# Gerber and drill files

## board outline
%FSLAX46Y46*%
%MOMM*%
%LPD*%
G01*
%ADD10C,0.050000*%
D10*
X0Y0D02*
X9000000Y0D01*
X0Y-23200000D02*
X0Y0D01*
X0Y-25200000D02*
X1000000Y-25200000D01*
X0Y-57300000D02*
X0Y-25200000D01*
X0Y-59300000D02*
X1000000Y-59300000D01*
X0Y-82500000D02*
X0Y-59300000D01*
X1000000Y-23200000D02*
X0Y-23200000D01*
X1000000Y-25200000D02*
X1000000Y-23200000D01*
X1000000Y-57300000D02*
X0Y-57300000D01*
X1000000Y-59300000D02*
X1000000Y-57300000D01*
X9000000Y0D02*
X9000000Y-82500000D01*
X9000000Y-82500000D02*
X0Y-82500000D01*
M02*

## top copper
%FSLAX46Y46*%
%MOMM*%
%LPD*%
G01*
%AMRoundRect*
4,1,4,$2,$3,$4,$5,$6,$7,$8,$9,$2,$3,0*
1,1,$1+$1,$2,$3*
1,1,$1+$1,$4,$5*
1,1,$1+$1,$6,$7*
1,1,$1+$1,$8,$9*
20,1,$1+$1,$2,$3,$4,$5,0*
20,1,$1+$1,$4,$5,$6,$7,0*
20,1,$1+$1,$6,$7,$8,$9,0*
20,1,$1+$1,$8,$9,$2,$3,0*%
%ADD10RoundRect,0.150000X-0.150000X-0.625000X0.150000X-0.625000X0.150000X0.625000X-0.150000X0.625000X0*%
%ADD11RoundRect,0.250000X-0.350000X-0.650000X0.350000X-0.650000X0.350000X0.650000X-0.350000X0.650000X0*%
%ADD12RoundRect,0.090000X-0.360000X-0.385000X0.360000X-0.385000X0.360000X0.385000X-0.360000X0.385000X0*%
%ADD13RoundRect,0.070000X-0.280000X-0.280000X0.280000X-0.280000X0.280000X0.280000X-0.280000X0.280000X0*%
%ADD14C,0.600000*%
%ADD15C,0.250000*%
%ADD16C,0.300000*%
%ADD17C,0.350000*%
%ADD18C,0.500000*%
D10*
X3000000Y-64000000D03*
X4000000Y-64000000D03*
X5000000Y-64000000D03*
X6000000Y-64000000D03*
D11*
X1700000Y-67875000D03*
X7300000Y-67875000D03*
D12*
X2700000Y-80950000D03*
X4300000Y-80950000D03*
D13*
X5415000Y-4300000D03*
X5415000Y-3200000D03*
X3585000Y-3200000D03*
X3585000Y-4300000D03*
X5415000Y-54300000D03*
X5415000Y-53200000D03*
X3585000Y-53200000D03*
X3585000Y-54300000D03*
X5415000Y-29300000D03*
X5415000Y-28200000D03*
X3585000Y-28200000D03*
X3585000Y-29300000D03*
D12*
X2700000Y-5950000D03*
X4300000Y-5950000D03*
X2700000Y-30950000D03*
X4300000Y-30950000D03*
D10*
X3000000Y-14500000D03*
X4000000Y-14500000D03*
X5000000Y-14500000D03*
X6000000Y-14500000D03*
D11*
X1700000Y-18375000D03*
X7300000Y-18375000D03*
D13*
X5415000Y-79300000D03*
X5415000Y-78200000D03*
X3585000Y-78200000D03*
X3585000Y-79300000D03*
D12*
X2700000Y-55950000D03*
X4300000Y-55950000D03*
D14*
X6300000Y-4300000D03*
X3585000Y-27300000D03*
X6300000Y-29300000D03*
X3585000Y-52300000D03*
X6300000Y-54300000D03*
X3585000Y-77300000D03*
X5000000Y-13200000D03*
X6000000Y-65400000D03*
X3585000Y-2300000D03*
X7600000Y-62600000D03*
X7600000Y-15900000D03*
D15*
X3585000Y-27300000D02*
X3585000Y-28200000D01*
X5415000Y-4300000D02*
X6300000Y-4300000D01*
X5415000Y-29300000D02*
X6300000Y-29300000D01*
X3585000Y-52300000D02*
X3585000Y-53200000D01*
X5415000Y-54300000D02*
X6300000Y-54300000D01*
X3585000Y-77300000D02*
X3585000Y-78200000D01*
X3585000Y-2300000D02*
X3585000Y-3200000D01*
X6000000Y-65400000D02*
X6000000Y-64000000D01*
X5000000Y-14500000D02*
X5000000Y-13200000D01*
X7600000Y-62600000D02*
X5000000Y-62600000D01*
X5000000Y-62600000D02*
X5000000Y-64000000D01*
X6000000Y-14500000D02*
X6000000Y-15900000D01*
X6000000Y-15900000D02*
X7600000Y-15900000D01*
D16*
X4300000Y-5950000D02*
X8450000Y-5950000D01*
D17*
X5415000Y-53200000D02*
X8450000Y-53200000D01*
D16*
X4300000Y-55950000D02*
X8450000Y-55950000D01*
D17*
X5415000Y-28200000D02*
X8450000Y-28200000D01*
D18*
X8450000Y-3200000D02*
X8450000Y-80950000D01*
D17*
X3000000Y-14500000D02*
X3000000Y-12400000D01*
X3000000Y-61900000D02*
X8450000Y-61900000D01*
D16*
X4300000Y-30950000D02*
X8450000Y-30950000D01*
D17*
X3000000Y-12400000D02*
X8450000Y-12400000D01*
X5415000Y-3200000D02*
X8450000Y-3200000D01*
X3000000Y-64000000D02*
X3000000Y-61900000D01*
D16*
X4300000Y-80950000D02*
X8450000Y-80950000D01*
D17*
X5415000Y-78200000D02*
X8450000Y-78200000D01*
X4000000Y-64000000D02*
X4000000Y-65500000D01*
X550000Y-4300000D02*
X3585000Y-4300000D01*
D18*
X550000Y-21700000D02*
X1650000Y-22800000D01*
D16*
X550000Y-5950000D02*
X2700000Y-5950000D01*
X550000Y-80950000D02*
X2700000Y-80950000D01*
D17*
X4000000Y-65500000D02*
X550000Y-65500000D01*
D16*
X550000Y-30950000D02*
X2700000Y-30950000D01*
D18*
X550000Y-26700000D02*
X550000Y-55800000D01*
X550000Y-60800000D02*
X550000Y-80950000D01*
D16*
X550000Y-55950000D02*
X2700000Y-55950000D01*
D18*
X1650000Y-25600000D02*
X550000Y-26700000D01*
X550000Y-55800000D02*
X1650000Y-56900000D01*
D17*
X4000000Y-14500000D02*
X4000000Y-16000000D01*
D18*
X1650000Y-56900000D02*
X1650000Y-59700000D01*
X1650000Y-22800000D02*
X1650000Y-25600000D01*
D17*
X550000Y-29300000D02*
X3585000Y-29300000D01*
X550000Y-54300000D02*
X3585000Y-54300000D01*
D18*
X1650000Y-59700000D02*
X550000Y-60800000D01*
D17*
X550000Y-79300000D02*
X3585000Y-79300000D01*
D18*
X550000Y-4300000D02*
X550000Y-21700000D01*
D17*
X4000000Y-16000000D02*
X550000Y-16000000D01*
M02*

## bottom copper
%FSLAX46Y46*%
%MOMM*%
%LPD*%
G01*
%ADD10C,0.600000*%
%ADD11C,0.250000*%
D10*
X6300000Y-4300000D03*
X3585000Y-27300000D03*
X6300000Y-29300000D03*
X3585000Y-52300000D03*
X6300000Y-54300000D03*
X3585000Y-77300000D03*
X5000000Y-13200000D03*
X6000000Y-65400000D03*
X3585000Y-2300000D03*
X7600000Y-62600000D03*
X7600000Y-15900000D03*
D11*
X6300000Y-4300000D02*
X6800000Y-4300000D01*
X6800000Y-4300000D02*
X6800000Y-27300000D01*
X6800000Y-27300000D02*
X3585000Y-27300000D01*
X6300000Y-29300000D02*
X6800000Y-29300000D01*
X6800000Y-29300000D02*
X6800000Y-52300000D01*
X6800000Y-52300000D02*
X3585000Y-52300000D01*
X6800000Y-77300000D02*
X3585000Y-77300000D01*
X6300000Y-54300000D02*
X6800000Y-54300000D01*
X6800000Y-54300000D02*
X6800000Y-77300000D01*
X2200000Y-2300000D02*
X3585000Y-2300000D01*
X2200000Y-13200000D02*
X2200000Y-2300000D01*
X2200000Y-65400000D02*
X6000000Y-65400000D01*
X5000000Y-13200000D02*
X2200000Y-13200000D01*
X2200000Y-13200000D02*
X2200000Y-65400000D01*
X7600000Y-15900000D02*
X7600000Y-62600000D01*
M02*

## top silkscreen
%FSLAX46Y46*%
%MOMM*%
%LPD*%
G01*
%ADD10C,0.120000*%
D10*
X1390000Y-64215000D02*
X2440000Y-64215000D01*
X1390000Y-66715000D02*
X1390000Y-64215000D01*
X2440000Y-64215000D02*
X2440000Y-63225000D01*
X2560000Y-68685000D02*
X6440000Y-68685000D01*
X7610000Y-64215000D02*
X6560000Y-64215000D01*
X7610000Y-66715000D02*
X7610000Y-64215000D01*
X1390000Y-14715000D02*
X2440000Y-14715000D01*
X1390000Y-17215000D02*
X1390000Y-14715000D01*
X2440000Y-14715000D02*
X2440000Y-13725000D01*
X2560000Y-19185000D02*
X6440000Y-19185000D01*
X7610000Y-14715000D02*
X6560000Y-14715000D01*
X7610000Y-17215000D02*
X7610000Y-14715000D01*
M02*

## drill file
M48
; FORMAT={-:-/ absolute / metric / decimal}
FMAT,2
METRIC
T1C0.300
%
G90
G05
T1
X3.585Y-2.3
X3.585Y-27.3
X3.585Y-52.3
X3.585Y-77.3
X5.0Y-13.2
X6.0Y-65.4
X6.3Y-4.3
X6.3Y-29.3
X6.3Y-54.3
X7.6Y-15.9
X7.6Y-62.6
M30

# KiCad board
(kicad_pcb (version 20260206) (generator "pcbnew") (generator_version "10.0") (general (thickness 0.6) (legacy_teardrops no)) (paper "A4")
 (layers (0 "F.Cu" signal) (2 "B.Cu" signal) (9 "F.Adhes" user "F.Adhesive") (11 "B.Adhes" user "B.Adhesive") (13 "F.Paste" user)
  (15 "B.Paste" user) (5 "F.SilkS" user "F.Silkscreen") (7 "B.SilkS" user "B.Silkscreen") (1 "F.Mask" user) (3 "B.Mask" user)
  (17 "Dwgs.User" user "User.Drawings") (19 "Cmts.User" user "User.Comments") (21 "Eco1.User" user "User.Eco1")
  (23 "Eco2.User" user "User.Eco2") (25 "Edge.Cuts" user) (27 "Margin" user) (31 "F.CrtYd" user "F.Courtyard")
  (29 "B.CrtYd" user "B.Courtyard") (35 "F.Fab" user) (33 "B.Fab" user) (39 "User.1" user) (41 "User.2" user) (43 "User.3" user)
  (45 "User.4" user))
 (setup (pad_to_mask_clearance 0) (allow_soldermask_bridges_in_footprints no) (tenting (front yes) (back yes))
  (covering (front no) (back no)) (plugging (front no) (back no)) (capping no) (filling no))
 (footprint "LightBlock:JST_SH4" (layer "F.Cu") (at 4.5 66)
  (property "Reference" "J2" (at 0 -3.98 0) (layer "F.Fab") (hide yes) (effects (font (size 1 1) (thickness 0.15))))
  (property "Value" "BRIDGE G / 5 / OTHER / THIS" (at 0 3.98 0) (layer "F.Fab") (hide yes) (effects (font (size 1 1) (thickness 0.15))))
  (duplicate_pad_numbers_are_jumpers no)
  (fp_line (start -3.11 -1.785) (end -2.06 -1.785) (stroke (width 0.12) (type solid)) (layer "F.SilkS"))
  (fp_line (start -3.11 0.715) (end -3.11 -1.785) (stroke (width 0.12) (type solid)) (layer "F.SilkS"))
  (fp_line (start -2.06 -1.785) (end -2.06 -2.775) (stroke (width 0.12) (type solid)) (layer "F.SilkS"))
  (fp_line (start -1.94 2.685) (end 1.94 2.685) (stroke (width 0.12) (type solid)) (layer "F.SilkS"))
  (fp_line (start 3.11 -1.785) (end 2.06 -1.785) (stroke (width 0.12) (type solid)) (layer "F.SilkS"))
  (fp_line (start 3.11 0.715) (end 3.11 -1.785) (stroke (width 0.12) (type solid)) (layer "F.SilkS"))
  (pad "1" smd roundrect (at -1.5 -2) (size 0.6 1.55) (layers "F.Cu" "F.Mask" "F.Paste") (roundrect_rratio 0.25) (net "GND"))
  (pad "2" smd roundrect (at -0.5 -2) (size 0.6 1.55) (layers "F.Cu" "F.Mask" "F.Paste") (roundrect_rratio 0.25) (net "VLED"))
  (pad "3" smd roundrect (at 0.5 -2) (size 0.6 1.55) (layers "F.Cu" "F.Mask" "F.Paste") (roundrect_rratio 0.25) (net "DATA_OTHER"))
  (pad "4" smd roundrect (at 1.5 -2) (size 0.6 1.55) (layers "F.Cu" "F.Mask" "F.Paste") (roundrect_rratio 0.25) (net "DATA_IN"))
  (pad "MP" smd roundrect (at -2.8 1.875) (size 1.2 1.8) (layers "F.Cu" "F.Mask" "F.Paste") (roundrect_rratio 0.208333))
  (pad "MP" smd roundrect (at 2.8 1.875) (size 1.2 1.8) (layers "F.Cu" "F.Mask" "F.Paste") (roundrect_rratio 0.208333)))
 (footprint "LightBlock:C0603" (layer "F.Cu") (at 3.5 80.95)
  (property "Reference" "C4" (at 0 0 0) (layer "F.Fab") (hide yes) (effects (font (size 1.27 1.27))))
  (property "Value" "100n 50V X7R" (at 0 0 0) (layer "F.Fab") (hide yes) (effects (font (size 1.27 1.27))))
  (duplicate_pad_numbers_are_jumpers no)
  (pad "1" smd roundrect (at -0.8 0) (size 0.9 0.95) (layers "F.Cu" "F.Mask" "F.Paste") (roundrect_rratio 0.1) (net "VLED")
   (thermal_bridge_angle 45))
  (pad "2" smd roundrect (at 0.8 0) (size 0.9 0.95) (layers "F.Cu" "F.Mask" "F.Paste") (roundrect_rratio 0.1) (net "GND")
   (thermal_bridge_angle 45)))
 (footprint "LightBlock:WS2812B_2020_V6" (layer "F.Cu") (at 4.5 3.75)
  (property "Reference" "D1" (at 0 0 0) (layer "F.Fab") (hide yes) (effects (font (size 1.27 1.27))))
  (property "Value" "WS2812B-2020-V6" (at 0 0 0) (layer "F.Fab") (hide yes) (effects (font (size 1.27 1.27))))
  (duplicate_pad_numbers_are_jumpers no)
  (pad "1" smd roundrect (at 0.915 0.55) (size 0.7 0.7) (layers "F.Cu" "F.Mask" "F.Paste") (roundrect_rratio 0.1) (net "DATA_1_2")
   (thermal_bridge_angle 45))
  (pad "2" smd roundrect (at 0.915 -0.55) (size 0.7 0.7) (layers "F.Cu" "F.Mask" "F.Paste") (roundrect_rratio 0.1) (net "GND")
   (thermal_bridge_angle 45))
  (pad "3" smd roundrect (at -0.915 -0.55) (size 0.7 0.7) (layers "F.Cu" "F.Mask" "F.Paste") (roundrect_rratio 0.1) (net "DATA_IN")
   (thermal_bridge_angle 45))
  (pad "4" smd roundrect (at -0.915 0.55) (size 0.7 0.7) (layers "F.Cu" "F.Mask" "F.Paste") (roundrect_rratio 0.1) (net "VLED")
   (thermal_bridge_angle 45)))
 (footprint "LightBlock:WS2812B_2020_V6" (layer "F.Cu") (at 4.5 53.75)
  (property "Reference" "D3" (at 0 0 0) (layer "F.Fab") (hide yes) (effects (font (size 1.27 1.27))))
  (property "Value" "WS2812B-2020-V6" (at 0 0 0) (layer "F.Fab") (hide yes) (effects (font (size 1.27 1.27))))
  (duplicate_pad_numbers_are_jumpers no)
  (pad "1" smd roundrect (at 0.915 0.55) (size 0.7 0.7) (layers "F.Cu" "F.Mask" "F.Paste") (roundrect_rratio 0.1) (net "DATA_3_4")
   (thermal_bridge_angle 45))
  (pad "2" smd roundrect (at 0.915 -0.55) (size 0.7 0.7) (layers "F.Cu" "F.Mask" "F.Paste") (roundrect_rratio 0.1) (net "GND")
   (thermal_bridge_angle 45))
  (pad "3" smd roundrect (at -0.915 -0.55) (size 0.7 0.7) (layers "F.Cu" "F.Mask" "F.Paste") (roundrect_rratio 0.1) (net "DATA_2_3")
   (thermal_bridge_angle 45))
  (pad "4" smd roundrect (at -0.915 0.55) (size 0.7 0.7) (layers "F.Cu" "F.Mask" "F.Paste") (roundrect_rratio 0.1) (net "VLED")
   (thermal_bridge_angle 45)))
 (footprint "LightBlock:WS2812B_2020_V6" (layer "F.Cu") (at 4.5 28.75)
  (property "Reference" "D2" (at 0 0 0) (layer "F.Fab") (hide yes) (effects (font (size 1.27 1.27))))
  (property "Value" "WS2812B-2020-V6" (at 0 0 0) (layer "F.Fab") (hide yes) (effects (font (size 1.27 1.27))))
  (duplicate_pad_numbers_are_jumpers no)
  (pad "1" smd roundrect (at 0.915 0.55) (size 0.7 0.7) (layers "F.Cu" "F.Mask" "F.Paste") (roundrect_rratio 0.1) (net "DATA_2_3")
   (thermal_bridge_angle 45))
  (pad "2" smd roundrect (at 0.915 -0.55) (size 0.7 0.7) (layers "F.Cu" "F.Mask" "F.Paste") (roundrect_rratio 0.1) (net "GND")
   (thermal_bridge_angle 45))
  (pad "3" smd roundrect (at -0.915 -0.55) (size 0.7 0.7) (layers "F.Cu" "F.Mask" "F.Paste") (roundrect_rratio 0.1) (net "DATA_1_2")
   (thermal_bridge_angle 45))
  (pad "4" smd roundrect (at -0.915 0.55) (size 0.7 0.7) (layers "F.Cu" "F.Mask" "F.Paste") (roundrect_rratio 0.1) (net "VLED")
   (thermal_bridge_angle 45)))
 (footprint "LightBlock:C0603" (layer "F.Cu") (at 3.5 5.95)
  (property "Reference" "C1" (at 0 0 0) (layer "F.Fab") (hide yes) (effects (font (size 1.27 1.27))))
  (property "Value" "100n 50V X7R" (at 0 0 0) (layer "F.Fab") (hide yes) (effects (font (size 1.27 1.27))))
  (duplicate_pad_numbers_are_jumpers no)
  (pad "1" smd roundrect (at -0.8 0) (size 0.9 0.95) (layers "F.Cu" "F.Mask" "F.Paste") (roundrect_rratio 0.1) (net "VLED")
   (thermal_bridge_angle 45))
  (pad "2" smd roundrect (at 0.8 0) (size 0.9 0.95) (layers "F.Cu" "F.Mask" "F.Paste") (roundrect_rratio 0.1) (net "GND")
   (thermal_bridge_angle 45)))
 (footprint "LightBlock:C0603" (layer "F.Cu") (at 3.5 30.95)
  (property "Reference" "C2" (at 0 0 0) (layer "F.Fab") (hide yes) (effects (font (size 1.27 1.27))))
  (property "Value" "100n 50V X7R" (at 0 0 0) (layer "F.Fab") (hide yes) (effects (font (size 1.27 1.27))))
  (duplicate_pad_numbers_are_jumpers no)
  (pad "1" smd roundrect (at -0.8 0) (size 0.9 0.95) (layers "F.Cu" "F.Mask" "F.Paste") (roundrect_rratio 0.1) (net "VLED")
   (thermal_bridge_angle 45))
  (pad "2" smd roundrect (at 0.8 0) (size 0.9 0.95) (layers "F.Cu" "F.Mask" "F.Paste") (roundrect_rratio 0.1) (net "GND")
   (thermal_bridge_angle 45)))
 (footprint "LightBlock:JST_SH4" (layer "F.Cu") (at 4.5 16.5)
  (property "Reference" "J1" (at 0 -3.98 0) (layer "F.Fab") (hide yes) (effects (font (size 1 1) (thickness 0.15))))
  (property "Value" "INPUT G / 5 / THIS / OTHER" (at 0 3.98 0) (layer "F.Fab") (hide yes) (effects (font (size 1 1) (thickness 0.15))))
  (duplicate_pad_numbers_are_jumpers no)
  (fp_line (start -3.11 -1.785) (end -2.06 -1.785) (stroke (width 0.12) (type solid)) (layer "F.SilkS"))
  (fp_line (start -3.11 0.715) (end -3.11 -1.785) (stroke (width 0.12) (type solid)) (layer "F.SilkS"))
  (fp_line (start -2.06 -1.785) (end -2.06 -2.775) (stroke (width 0.12) (type solid)) (layer "F.SilkS"))
  (fp_line (start -1.94 2.685) (end 1.94 2.685) (stroke (width 0.12) (type solid)) (layer "F.SilkS"))
  (fp_line (start 3.11 -1.785) (end 2.06 -1.785) (stroke (width 0.12) (type solid)) (layer "F.SilkS"))
  (fp_line (start 3.11 0.715) (end 3.11 -1.785) (stroke (width 0.12) (type solid)) (layer "F.SilkS"))
  (pad "1" smd roundrect (at -1.5 -2) (size 0.6 1.55) (layers "F.Cu" "F.Mask" "F.Paste") (roundrect_rratio 0.25) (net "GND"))
  (pad "2" smd roundrect (at -0.5 -2) (size 0.6 1.55) (layers "F.Cu" "F.Mask" "F.Paste") (roundrect_rratio 0.25) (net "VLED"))
  (pad "3" smd roundrect (at 0.5 -2) (size 0.6 1.55) (layers "F.Cu" "F.Mask" "F.Paste") (roundrect_rratio 0.25) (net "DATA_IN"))
  (pad "4" smd roundrect (at 1.5 -2) (size 0.6 1.55) (layers "F.Cu" "F.Mask" "F.Paste") (roundrect_rratio 0.25) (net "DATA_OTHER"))
  (pad "MP" smd roundrect (at -2.8 1.875) (size 1.2 1.8) (layers "F.Cu" "F.Mask" "F.Paste") (roundrect_rratio 0.208333))
  (pad "MP" smd roundrect (at 2.8 1.875) (size 1.2 1.8) (layers "F.Cu" "F.Mask" "F.Paste") (roundrect_rratio 0.208333)))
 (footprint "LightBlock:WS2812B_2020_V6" (layer "F.Cu") (at 4.5 78.75)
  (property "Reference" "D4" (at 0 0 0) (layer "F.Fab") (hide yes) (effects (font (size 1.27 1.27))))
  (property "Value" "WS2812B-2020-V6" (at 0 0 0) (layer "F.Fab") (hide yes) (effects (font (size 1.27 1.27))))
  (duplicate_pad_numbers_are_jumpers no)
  (pad "1" smd roundrect (at 0.915 0.55) (size 0.7 0.7) (layers "F.Cu" "F.Mask" "F.Paste") (roundrect_rratio 0.1) (thermal_bridge_angle 45))
  (pad "2" smd roundrect (at 0.915 -0.55) (size 0.7 0.7) (layers "F.Cu" "F.Mask" "F.Paste") (roundrect_rratio 0.1) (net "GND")
   (thermal_bridge_angle 45))
  (pad "3" smd roundrect (at -0.915 -0.55) (size 0.7 0.7) (layers "F.Cu" "F.Mask" "F.Paste") (roundrect_rratio 0.1) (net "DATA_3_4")
   (thermal_bridge_angle 45))
  (pad "4" smd roundrect (at -0.915 0.55) (size 0.7 0.7) (layers "F.Cu" "F.Mask" "F.Paste") (roundrect_rratio 0.1) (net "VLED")
   (thermal_bridge_angle 45)))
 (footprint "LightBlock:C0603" (layer "F.Cu") (at 3.5 55.95)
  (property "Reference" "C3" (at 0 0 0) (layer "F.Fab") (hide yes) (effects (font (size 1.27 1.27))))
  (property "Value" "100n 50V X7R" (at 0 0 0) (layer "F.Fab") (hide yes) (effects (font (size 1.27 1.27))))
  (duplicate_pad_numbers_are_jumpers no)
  (pad "1" smd roundrect (at -0.8 0) (size 0.9 0.95) (layers "F.Cu" "F.Mask" "F.Paste") (roundrect_rratio 0.1) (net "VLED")
   (thermal_bridge_angle 45))
  (pad "2" smd roundrect (at 0.8 0) (size 0.9 0.95) (layers "F.Cu" "F.Mask" "F.Paste") (roundrect_rratio 0.1) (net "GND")
   (thermal_bridge_angle 45)))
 (gr_line (start 0 0) (end 9 0) (stroke (width 0.05) (type default)) (layer "Edge.Cuts"))
 (gr_line (start 0 23.2) (end 0 0) (stroke (width 0.05) (type default)) (layer "Edge.Cuts"))
 (gr_line (start 0 25.2) (end 1 25.2) (stroke (width 0.05) (type default)) (layer "Edge.Cuts"))
 (gr_line (start 0 57.3) (end 0 25.2) (stroke (width 0.05) (type default)) (layer "Edge.Cuts"))
 (gr_line (start 0 59.3) (end 1 59.3) (stroke (width 0.05) (type default)) (layer "Edge.Cuts"))
 (gr_line (start 0 82.5) (end 0 59.3) (stroke (width 0.05) (type default)) (layer "Edge.Cuts"))
 (gr_line (start 1 23.2) (end 0 23.2) (stroke (width 0.05) (type default)) (layer "Edge.Cuts"))
 (gr_line (start 1 25.2) (end 1 23.2) (stroke (width 0.05) (type default)) (layer "Edge.Cuts"))
 (gr_line (start 1 57.3) (end 0 57.3) (stroke (width 0.05) (type default)) (layer "Edge.Cuts"))
 (gr_line (start 1 59.3) (end 1 57.3) (stroke (width 0.05) (type default)) (layer "Edge.Cuts"))
 (gr_line (start 9 0) (end 9 82.5) (stroke (width 0.05) (type default)) (layer "Edge.Cuts"))
 (gr_line (start 9 82.5) (end 0 82.5) (stroke (width 0.05) (type default)) (layer "Edge.Cuts"))
 (segment (start 3.585 27.3) (end 3.585 28.2) (width 0.25) (layer "F.Cu") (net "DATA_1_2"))
 (segment (start 5.415 4.3) (end 6.3 4.3) (width 0.25) (layer "F.Cu") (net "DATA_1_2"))
 (via (at 6.3 4.3) (size 0.6) (drill 0.3) (layers "F.Cu" "B.Cu") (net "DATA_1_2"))
 (via (at 3.585 27.3) (size 0.6) (drill 0.3) (layers "F.Cu" "B.Cu") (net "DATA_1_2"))
 (segment (start 6.3 4.3) (end 6.8 4.3) (width 0.25) (layer "B.Cu") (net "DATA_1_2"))
 (segment (start 6.8 4.3) (end 6.8 27.3) (width 0.25) (layer "B.Cu") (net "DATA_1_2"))
 (segment (start 6.8 27.3) (end 3.585 27.3) (width 0.25) (layer "B.Cu") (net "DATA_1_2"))
 (segment (start 5.415 29.3) (end 6.3 29.3) (width 0.25) (layer "F.Cu") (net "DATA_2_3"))
 (segment (start 3.585 52.3) (end 3.585 53.2) (width 0.25) (layer "F.Cu") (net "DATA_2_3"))
 (via (at 6.3 29.3) (size 0.6) (drill 0.3) (layers "F.Cu" "B.Cu") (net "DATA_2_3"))
 (via (at 3.585 52.3) (size 0.6) (drill 0.3) (layers "F.Cu" "B.Cu") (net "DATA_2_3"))
 (segment (start 6.3 29.3) (end 6.8 29.3) (width 0.25) (layer "B.Cu") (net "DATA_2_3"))
 (segment (start 6.8 29.3) (end 6.8 52.3) (width 0.25) (layer "B.Cu") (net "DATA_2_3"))
 (segment (start 6.8 52.3) (end 3.585 52.3) (width 0.25) (layer "B.Cu") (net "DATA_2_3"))
 (segment (start 5.415 54.3) (end 6.3 54.3) (width 0.25) (layer "F.Cu") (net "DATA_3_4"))
 (segment (start 3.585 77.3) (end 3.585 78.2) (width 0.25) (layer "F.Cu") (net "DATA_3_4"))
 (via (at 6.3 54.3) (size 0.6) (drill 0.3) (layers "F.Cu" "B.Cu") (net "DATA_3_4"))
 (via (at 3.585 77.3) (size 0.6) (drill 0.3) (layers "F.Cu" "B.Cu") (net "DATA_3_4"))
 (segment (start 6.8 77.3) (end 3.585 77.3) (width 0.25) (layer "B.Cu") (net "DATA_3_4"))
 (segment (start 6.3 54.3) (end 6.8 54.3) (width 0.25) (layer "B.Cu") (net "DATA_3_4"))
 (segment (start 6.8 54.3) (end 6.8 77.3) (width 0.25) (layer "B.Cu") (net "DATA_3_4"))
 (segment (start 3.585 2.3) (end 3.585 3.2) (width 0.25) (layer "F.Cu") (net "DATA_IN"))
 (segment (start 6 65.4) (end 6 64) (width 0.25) (layer "F.Cu") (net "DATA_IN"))
 (segment (start 5 14.5) (end 5 13.2) (width 0.25) (layer "F.Cu") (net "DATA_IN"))
 (via (at 5 13.2) (size 0.6) (drill 0.3) (layers "F.Cu" "B.Cu") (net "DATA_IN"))
 (via (at 6 65.4) (size 0.6) (drill 0.3) (layers "F.Cu" "B.Cu") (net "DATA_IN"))
 (via (at 3.585 2.3) (size 0.6) (drill 0.3) (layers "F.Cu" "B.Cu") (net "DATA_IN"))
 (segment (start 2.2 2.3) (end 3.585 2.3) (width 0.25) (layer "B.Cu") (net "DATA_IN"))
 (segment (start 2.2 13.2) (end 2.2 2.3) (width 0.25) (layer "B.Cu") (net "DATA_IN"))
 (segment (start 2.2 65.4) (end 6 65.4) (width 0.25) (layer "B.Cu") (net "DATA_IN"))
 (segment (start 5 13.2) (end 2.2 13.2) (width 0.25) (layer "B.Cu") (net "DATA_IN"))
 (segment (start 2.2 13.2) (end 2.2 65.4) (width 0.25) (layer "B.Cu") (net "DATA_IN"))
 (segment (start 7.6 62.6) (end 5 62.6) (width 0.25) (layer "F.Cu") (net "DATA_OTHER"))
 (segment (start 5 62.6) (end 5 64) (width 0.25) (layer "F.Cu") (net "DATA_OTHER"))
 (segment (start 6 14.5) (end 6 15.9) (width 0.25) (layer "F.Cu") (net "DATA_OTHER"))
 (segment (start 6 15.9) (end 7.6 15.9) (width 0.25) (layer "F.Cu") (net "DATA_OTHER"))
 (via (at 7.6 62.6) (size 0.6) (drill 0.3) (layers "F.Cu" "B.Cu") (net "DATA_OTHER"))
 (via (at 7.6 15.9) (size 0.6) (drill 0.3) (layers "F.Cu" "B.Cu") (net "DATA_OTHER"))
 (segment (start 7.6 15.9) (end 7.6 62.6) (width 0.25) (layer "B.Cu") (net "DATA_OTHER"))
 (segment (start 4.3 5.95) (end 8.45 5.95) (width 0.3) (layer "F.Cu") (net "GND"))
 (segment (start 5.415 53.2) (end 8.45 53.2) (width 0.35) (layer "F.Cu") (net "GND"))
 (segment (start 4.3 55.95) (end 8.45 55.95) (width 0.3) (layer "F.Cu") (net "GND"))
 (segment (start 5.415 28.2) (end 8.45 28.2) (width 0.35) (layer "F.Cu") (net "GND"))
 (segment (start 8.45 3.2) (end 8.45 80.95) (width 0.5) (layer "F.Cu") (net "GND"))
 (segment (start 3 14.5) (end 3 12.4) (width 0.35) (layer "F.Cu") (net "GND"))
 (segment (start 3 61.9) (end 8.45 61.9) (width 0.35) (layer "F.Cu") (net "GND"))
 (segment (start 4.3 30.95) (end 8.45 30.95) (width 0.3) (layer "F.Cu") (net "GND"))
 (segment (start 3 12.4) (end 8.45 12.4) (width 0.35) (layer "F.Cu") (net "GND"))
 (segment (start 5.415 3.2) (end 8.45 3.2) (width 0.35) (layer "F.Cu") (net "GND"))
 (segment (start 3 64) (end 3 61.9) (width 0.35) (layer "F.Cu") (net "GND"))
 (segment (start 4.3 80.95) (end 8.45 80.95) (width 0.3) (layer "F.Cu") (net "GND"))
 (segment (start 5.415 78.2) (end 8.45 78.2) (width 0.35) (layer "F.Cu") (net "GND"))
 (segment (start 4 64) (end 4 65.5) (width 0.35) (layer "F.Cu") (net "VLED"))
 (segment (start 0.55 4.3) (end 3.585 4.3) (width 0.35) (layer "F.Cu") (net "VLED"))
 (segment (start 0.55 21.7) (end 1.65 22.8) (width 0.5) (layer "F.Cu") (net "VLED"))
 (segment (start 0.55 5.95) (end 2.7 5.95) (width 0.3) (layer "F.Cu") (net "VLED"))
 (segment (start 0.55 80.95) (end 2.7 80.95) (width 0.3) (layer "F.Cu") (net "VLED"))
 (segment (start 4 65.5) (end 0.55 65.5) (width 0.35) (layer "F.Cu") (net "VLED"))
 (segment (start 0.55 30.95) (end 2.7 30.95) (width 0.3) (layer "F.Cu") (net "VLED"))
 (segment (start 0.55 26.7) (end 0.55 55.8) (width 0.5) (layer "F.Cu") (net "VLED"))
 (segment (start 0.55 60.8) (end 0.55 80.95) (width 0.5) (layer "F.Cu") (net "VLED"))
 (segment (start 0.55 55.95) (end 2.7 55.95) (width 0.3) (layer "F.Cu") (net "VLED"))
 (segment (start 1.65 25.6) (end 0.55 26.7) (width 0.5) (layer "F.Cu") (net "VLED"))
 (segment (start 0.55 55.8) (end 1.65 56.9) (width 0.5) (layer "F.Cu") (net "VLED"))
 (segment (start 4 14.5) (end 4 16) (width 0.35) (layer "F.Cu") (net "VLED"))
 (segment (start 1.65 56.9) (end 1.65 59.7) (width 0.5) (layer "F.Cu") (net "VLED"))
 (segment (start 1.65 22.8) (end 1.65 25.6) (width 0.5) (layer "F.Cu") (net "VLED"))
 (segment (start 0.55 29.3) (end 3.585 29.3) (width 0.35) (layer "F.Cu") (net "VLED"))
 (segment (start 0.55 54.3) (end 3.585 54.3) (width 0.35) (layer "F.Cu") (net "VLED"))
 (segment (start 1.65 59.7) (end 0.55 60.8) (width 0.5) (layer "F.Cu") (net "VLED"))
 (segment (start 0.55 79.3) (end 3.585 79.3) (width 0.35) (layer "F.Cu") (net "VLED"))
 (segment (start 0.55 4.3) (end 0.55 21.7) (width 0.5) (layer "F.Cu") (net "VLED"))
 (segment (start 4 16) (end 0.55 16) (width 0.35) (layer "F.Cu") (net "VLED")))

